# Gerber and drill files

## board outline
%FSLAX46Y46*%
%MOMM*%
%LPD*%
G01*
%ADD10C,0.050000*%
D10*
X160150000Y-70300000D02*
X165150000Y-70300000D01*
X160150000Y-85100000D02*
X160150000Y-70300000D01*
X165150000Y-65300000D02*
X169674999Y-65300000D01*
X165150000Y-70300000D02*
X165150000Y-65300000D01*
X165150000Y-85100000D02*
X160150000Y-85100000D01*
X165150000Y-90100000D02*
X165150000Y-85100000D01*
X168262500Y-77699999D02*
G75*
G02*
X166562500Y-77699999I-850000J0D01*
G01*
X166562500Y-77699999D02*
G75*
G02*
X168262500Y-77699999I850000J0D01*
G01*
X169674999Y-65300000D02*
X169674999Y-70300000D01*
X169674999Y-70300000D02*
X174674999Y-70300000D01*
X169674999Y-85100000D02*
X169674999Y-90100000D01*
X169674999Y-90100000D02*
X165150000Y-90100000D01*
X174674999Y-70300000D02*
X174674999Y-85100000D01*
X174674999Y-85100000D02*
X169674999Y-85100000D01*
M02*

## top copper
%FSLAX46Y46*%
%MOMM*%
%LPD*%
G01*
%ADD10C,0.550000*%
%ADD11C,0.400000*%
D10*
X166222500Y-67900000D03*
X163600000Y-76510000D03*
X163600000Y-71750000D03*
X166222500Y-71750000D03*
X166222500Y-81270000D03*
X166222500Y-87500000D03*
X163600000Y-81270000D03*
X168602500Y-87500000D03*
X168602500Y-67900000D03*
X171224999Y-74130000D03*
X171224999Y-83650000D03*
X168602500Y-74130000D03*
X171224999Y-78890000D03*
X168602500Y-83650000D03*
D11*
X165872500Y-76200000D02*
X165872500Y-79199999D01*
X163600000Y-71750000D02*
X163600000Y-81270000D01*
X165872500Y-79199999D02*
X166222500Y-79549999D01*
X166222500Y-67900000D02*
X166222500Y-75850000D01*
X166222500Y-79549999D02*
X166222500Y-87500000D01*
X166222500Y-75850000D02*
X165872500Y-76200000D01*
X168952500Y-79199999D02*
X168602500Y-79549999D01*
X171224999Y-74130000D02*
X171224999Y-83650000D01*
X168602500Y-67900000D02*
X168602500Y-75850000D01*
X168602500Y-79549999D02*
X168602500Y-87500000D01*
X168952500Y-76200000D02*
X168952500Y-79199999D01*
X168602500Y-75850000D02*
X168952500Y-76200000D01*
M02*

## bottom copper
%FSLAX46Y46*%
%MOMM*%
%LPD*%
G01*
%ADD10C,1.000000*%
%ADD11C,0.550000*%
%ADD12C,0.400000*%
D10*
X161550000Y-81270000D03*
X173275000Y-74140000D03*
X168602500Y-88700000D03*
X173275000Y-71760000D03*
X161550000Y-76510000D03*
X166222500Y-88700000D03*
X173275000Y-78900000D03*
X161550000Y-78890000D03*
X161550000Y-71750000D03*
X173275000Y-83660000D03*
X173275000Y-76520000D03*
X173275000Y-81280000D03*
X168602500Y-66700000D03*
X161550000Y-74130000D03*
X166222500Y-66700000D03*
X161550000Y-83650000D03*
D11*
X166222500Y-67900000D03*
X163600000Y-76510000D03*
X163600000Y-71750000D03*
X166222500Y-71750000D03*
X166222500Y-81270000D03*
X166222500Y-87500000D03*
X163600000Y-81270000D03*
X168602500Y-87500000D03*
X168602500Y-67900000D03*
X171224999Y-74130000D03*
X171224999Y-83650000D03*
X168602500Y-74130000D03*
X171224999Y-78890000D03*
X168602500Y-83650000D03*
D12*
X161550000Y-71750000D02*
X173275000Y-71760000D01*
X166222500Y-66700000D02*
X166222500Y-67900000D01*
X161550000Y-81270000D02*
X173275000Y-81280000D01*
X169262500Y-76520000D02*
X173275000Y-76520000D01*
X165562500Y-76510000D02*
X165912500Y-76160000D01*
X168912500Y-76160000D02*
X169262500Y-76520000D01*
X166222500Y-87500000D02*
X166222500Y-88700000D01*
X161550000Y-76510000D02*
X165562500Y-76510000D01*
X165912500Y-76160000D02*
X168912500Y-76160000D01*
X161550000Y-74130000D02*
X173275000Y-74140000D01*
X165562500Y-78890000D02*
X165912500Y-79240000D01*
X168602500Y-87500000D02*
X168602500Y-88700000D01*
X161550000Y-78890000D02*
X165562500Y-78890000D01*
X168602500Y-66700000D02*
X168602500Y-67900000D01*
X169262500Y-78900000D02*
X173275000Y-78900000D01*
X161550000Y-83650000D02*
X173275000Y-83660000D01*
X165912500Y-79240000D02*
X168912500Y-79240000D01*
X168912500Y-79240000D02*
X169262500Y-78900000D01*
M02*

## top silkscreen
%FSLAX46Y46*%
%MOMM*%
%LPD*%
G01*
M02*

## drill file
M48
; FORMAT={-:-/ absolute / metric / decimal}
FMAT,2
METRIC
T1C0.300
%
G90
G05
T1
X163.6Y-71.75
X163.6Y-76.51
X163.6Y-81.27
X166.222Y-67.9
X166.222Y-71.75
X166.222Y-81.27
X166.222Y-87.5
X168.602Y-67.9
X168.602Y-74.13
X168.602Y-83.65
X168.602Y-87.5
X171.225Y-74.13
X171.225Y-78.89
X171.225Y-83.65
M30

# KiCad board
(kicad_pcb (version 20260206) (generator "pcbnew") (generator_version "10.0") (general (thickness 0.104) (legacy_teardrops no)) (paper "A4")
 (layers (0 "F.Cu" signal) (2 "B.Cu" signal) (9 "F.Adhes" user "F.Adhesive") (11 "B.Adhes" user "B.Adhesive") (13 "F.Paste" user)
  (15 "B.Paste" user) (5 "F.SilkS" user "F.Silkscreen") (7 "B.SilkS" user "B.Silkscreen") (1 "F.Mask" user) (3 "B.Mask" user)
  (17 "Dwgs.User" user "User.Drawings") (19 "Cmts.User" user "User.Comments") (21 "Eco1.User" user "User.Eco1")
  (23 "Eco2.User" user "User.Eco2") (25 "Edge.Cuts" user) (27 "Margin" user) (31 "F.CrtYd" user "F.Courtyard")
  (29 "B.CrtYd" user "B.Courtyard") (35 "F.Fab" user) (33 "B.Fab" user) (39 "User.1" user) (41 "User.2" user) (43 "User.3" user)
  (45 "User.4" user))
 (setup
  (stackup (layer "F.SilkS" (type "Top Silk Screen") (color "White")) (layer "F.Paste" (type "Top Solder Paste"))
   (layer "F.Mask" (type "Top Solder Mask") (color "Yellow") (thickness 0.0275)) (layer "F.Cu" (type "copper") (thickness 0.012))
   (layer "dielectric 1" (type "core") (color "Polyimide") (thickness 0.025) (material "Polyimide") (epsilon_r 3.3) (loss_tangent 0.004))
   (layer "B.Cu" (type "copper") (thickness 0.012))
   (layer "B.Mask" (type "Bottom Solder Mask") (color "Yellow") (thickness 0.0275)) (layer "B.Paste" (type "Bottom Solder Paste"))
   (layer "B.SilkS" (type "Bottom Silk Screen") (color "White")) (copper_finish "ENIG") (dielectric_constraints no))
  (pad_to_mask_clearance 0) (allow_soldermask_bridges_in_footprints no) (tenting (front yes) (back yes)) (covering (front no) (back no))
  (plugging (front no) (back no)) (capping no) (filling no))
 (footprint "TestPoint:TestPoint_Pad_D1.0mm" (layer "B.Cu") (at 161.55 81.27 -90)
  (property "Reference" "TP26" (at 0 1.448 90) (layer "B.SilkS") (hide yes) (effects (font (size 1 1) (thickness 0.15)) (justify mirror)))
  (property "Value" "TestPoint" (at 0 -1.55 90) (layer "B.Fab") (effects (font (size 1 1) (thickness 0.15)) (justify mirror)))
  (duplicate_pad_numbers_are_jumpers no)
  (pad "1" smd circle (at 0 0 270) (size 1 1) (layers "B.Cu" "B.Mask") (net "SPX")))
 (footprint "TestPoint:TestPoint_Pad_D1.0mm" (layer "B.Cu") (at 173.275 74.14 90)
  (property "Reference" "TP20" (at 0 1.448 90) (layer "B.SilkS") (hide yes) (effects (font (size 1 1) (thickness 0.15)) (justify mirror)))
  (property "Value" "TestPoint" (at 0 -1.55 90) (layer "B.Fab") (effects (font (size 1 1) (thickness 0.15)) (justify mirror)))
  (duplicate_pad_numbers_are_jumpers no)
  (pad "1" smd circle (at 0 0 90) (size 1 1) (layers "B.Cu" "B.Mask") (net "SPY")))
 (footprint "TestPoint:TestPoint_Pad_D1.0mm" (layer "B.Cu") (at 168.6025 88.7)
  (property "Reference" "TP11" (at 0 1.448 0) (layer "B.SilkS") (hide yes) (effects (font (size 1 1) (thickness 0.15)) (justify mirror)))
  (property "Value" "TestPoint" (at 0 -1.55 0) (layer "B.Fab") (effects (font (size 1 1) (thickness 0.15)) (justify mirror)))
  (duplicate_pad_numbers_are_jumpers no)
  (pad "1" smd circle (at 0 0) (size 1 1) (layers "B.Cu" "B.Mask") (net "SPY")))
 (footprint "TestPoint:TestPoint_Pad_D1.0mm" (layer "B.Cu") (at 173.275 71.76 90)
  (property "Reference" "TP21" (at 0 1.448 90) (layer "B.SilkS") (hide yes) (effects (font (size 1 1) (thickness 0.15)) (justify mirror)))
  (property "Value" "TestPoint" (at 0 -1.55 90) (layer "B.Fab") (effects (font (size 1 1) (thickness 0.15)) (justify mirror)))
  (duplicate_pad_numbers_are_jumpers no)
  (pad "1" smd circle (at 0 0 90) (size 1 1) (layers "B.Cu" "B.Mask") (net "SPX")))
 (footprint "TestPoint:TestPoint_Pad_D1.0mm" (layer "B.Cu") (at 161.55 76.51 -90)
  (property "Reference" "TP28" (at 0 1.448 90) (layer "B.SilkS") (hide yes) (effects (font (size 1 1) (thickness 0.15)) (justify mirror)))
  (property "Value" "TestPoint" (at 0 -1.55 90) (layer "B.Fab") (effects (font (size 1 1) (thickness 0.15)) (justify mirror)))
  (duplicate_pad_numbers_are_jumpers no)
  (pad "1" smd circle (at 0 0 270) (size 1 1) (layers "B.Cu" "B.Mask") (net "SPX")))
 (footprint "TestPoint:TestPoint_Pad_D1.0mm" (layer "B.Cu") (at 166.2225 88.7)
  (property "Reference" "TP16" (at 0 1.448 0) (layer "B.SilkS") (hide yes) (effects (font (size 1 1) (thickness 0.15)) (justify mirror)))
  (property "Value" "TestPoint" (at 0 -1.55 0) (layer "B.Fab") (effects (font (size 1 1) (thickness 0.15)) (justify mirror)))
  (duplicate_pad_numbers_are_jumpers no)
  (pad "1" smd circle (at 0 0) (size 1 1) (layers "B.Cu" "B.Mask") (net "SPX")))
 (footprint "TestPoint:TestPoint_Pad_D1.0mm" (layer "B.Cu") (at 173.275 78.9 90)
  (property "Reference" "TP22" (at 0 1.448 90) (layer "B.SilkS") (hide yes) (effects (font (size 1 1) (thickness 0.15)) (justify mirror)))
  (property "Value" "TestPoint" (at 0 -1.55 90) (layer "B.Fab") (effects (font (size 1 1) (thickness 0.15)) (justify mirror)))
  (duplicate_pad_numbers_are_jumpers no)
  (pad "1" smd circle (at 0 0 90) (size 1 1) (layers "B.Cu" "B.Mask") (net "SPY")))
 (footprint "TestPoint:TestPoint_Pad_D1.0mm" (layer "B.Cu") (at 161.55 78.89 -90)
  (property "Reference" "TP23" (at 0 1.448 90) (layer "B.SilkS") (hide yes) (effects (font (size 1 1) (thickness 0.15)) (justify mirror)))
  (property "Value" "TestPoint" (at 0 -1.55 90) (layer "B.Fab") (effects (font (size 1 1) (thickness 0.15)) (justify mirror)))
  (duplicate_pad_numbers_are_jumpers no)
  (pad "1" smd circle (at 0 0 270) (size 1 1) (layers "B.Cu" "B.Mask") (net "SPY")))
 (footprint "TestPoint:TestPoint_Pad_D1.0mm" (layer "B.Cu") (at 161.55 71.75 -90)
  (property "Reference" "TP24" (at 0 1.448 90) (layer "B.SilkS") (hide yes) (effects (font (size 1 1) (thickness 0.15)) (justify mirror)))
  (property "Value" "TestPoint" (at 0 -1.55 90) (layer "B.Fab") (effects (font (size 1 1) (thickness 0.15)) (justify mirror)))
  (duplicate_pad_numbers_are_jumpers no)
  (pad "1" smd circle (at 0 0 270) (size 1 1) (layers "B.Cu" "B.Mask") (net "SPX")))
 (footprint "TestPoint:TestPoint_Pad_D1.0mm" (layer "B.Cu") (at 173.275 83.66 90)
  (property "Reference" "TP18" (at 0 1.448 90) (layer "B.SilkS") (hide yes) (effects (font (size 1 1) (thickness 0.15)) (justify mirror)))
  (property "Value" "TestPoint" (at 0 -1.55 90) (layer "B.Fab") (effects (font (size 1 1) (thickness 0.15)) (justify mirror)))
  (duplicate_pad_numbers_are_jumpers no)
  (pad "1" smd circle (at 0 0 90) (size 1 1) (layers "B.Cu" "B.Mask") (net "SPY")))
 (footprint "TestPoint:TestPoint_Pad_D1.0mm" (layer "B.Cu") (at 173.275 76.52 90)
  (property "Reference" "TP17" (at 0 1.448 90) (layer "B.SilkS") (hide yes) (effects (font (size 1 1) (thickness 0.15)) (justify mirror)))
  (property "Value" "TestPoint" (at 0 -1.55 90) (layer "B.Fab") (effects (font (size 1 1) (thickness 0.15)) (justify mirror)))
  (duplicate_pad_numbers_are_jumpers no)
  (pad "1" smd circle (at 0 0 90) (size 1 1) (layers "B.Cu" "B.Mask") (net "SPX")))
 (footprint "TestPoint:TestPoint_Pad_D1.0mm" (layer "B.Cu") (at 173.275 81.28 90)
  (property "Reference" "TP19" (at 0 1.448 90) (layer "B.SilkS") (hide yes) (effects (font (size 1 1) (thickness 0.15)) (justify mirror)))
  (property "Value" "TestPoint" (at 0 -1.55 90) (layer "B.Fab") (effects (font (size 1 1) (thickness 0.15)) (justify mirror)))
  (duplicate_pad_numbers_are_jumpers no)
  (pad "1" smd circle (at 0 0 90) (size 1 1) (layers "B.Cu" "B.Mask") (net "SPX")))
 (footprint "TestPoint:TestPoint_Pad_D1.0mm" (layer "B.Cu") (at 168.6025 66.7 180)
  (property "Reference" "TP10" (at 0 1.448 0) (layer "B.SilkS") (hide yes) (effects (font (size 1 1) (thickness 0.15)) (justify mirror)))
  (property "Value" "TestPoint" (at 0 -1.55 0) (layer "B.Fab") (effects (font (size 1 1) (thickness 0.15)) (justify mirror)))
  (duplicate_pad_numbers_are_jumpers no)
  (pad "1" smd circle (at 0 0 180) (size 1 1) (layers "B.Cu" "B.Mask") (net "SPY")))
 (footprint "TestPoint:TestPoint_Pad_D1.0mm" (layer "B.Cu") (at 161.55 74.13 -90)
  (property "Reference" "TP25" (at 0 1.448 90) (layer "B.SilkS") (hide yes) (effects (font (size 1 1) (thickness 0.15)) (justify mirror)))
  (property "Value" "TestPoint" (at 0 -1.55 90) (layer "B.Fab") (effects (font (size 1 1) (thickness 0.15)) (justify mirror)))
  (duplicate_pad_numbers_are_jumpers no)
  (pad "1" smd circle (at 0 0 270) (size 1 1) (layers "B.Cu" "B.Mask") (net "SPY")))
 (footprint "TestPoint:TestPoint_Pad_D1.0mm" (layer "B.Cu") (at 166.2225 66.7 180)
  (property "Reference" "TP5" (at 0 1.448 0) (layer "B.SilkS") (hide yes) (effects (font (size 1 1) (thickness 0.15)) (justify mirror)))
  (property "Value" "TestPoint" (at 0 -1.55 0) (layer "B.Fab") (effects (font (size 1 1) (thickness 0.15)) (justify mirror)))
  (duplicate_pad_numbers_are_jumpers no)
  (pad "1" smd circle (at 0 0 180) (size 1 1) (layers "B.Cu" "B.Mask") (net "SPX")))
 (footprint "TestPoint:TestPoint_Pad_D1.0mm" (layer "B.Cu") (at 161.55 83.65 -90)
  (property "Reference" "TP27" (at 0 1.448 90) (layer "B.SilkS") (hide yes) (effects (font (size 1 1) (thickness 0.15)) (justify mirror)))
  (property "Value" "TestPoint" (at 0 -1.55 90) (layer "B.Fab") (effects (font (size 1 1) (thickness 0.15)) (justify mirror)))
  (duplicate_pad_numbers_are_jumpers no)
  (pad "1" smd circle (at 0 0 270) (size 1 1) (layers "B.Cu" "B.Mask") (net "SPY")))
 (gr_line (start 160.15 70.3) (end 165.15 70.3) (stroke (width 0.05) (type default)) (layer "Edge.Cuts"))
 (gr_line (start 160.15 85.1) (end 160.15 70.3) (stroke (width 0.05) (type default)) (layer "Edge.Cuts"))
 (gr_line (start 165.15 65.3) (end 169.674999 65.3) (stroke (width 0.05) (type default)) (layer "Edge.Cuts"))
 (gr_line (start 165.15 70.3) (end 165.15 65.3) (stroke (width 0.05) (type default)) (layer "Edge.Cuts"))
 (gr_line (start 165.15 85.1) (end 160.15 85.1) (stroke (width 0.05) (type default)) (layer "Edge.Cuts"))
 (gr_line (start 165.15 90.1) (end 165.15 85.1) (stroke (width 0.05) (type default)) (layer "Edge.Cuts"))
 (gr_circle (center 167.4125 77.699999) (end 168.2625 77.699999) (stroke (width 0.05) (type default)) (fill no) (layer "Edge.Cuts"))
 (gr_line (start 169.674999 65.3) (end 169.674999 70.3) (stroke (width 0.05) (type default)) (layer "Edge.Cuts"))
 (gr_line (start 169.674999 70.3) (end 174.674999 70.3) (stroke (width 0.05) (type default)) (layer "Edge.Cuts"))
 (gr_line (start 169.674999 85.1) (end 169.674999 90.1) (stroke (width 0.05) (type default)) (layer "Edge.Cuts"))
 (gr_line (start 169.674999 90.1) (end 165.15 90.1) (stroke (width 0.05) (type default)) (layer "Edge.Cuts"))
 (gr_line (start 174.674999 70.3) (end 174.674999 85.1) (stroke (width 0.05) (type default)) (layer "Edge.Cuts"))
 (gr_line (start 174.674999 85.1) (end 169.674999 85.1) (stroke (width 0.05) (type default)) (layer "Edge.Cuts"))
 (segment (start 165.8725 76.2) (end 165.8725 79.199999) (width 0.4) (layer "F.Cu") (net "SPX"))
 (segment (start 163.6 71.75) (end 163.6 81.27) (width 0.4) (layer "F.Cu") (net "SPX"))
 (segment (start 165.8725 79.199999) (end 166.2225 79.549999) (width 0.4) (layer "F.Cu") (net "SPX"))
 (segment (start 166.2225 67.9) (end 166.2225 75.85) (width 0.4) (layer "F.Cu") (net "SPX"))
 (segment (start 166.2225 79.549999) (end 166.2225 87.5) (width 0.4) (layer "F.Cu") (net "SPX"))
 (segment (start 166.2225 75.85) (end 165.8725 76.2) (width 0.4) (layer "F.Cu") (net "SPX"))
 (via (at 166.2225 67.9) (size 0.55) (drill 0.3) (layers "F.Cu" "B.Cu") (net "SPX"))
 (via (at 163.6 76.51) (size 0.55) (drill 0.3) (layers "F.Cu" "B.Cu") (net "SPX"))
 (via (at 163.6 71.75) (size 0.55) (drill 0.3) (layers "F.Cu" "B.Cu") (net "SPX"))
 (via (at 166.2225 71.75) (size 0.55) (drill 0.3) (layers "F.Cu" "B.Cu") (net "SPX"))
 (via (at 166.2225 81.27) (size 0.55) (drill 0.3) (layers "F.Cu" "B.Cu") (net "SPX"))
 (via (at 166.2225 87.5) (size 0.55) (drill 0.3) (layers "F.Cu" "B.Cu") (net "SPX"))
 (via (at 163.6 81.27) (size 0.55) (drill 0.3) (layers "F.Cu" "B.Cu") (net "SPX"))
 (segment (start 161.55 71.75) (end 173.275 71.76) (width 0.4) (layer "B.Cu") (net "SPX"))
 (segment (start 166.2225 66.7) (end 166.2225 67.9) (width 0.4) (layer "B.Cu") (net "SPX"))
 (segment (start 161.55 81.27) (end 173.275 81.28) (width 0.4) (layer "B.Cu") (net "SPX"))
 (segment (start 169.2625 76.52) (end 173.275 76.52) (width 0.4) (layer "B.Cu") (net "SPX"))
 (segment (start 165.5625 76.51) (end 165.9125 76.16) (width 0.4) (layer "B.Cu") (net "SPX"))
 (segment (start 168.9125 76.16) (end 169.2625 76.52) (width 0.4) (layer "B.Cu") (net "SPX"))
 (segment (start 166.2225 87.5) (end 166.2225 88.7) (width 0.4) (layer "B.Cu") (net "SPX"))
 (segment (start 161.55 76.51) (end 165.5625 76.51) (width 0.4) (layer "B.Cu") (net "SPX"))
 (segment (start 165.9125 76.16) (end 168.9125 76.16) (width 0.4) (layer "B.Cu") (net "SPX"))
 (segment (start 168.9525 79.199999) (end 168.6025 79.549999) (width 0.4) (layer "F.Cu") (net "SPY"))
 (segment (start 171.224999 74.13) (end 171.224999 83.65) (width 0.4) (layer "F.Cu") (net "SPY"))
 (segment (start 168.6025 67.9) (end 168.6025 75.85) (width 0.4) (layer "F.Cu") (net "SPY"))
 (segment (start 168.6025 79.549999) (end 168.6025 87.5) (width 0.4) (layer "F.Cu") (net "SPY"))
 (segment (start 168.9525 76.2) (end 168.9525 79.199999) (width 0.4) (layer "F.Cu") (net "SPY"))
 (segment (start 168.6025 75.85) (end 168.9525 76.2) (width 0.4) (layer "F.Cu") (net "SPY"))
 (via (at 168.6025 87.5) (size 0.55) (drill 0.3) (layers "F.Cu" "B.Cu") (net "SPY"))
 (via (at 168.6025 67.9) (size 0.55) (drill 0.3) (layers "F.Cu" "B.Cu") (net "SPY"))
 (via (at 171.224999 74.13) (size 0.55) (drill 0.3) (layers "F.Cu" "B.Cu") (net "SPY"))
 (via (at 171.224999 83.65) (size 0.55) (drill 0.3) (layers "F.Cu" "B.Cu") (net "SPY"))
 (via (at 168.6025 74.13) (size 0.55) (drill 0.3) (layers "F.Cu" "B.Cu") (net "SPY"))
 (via (at 171.224999 78.89) (size 0.55) (drill 0.3) (layers "F.Cu" "B.Cu") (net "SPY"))
 (via (at 168.6025 83.65) (size 0.55) (drill 0.3) (layers "F.Cu" "B.Cu") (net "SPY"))
 (segment (start 161.55 74.13) (end 173.275 74.14) (width 0.4) (layer "B.Cu") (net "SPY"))
 (segment (start 165.5625 78.89) (end 165.9125 79.24) (width 0.4) (layer "B.Cu") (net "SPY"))
 (segment (start 168.6025 87.5) (end 168.6025 88.7) (width 0.4) (layer "B.Cu") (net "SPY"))
 (segment (start 161.55 78.89) (end 165.5625 78.89) (width 0.4) (layer "B.Cu") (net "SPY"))
 (segment (start 168.6025 66.7) (end 168.6025 67.9) (width 0.4) (layer "B.Cu") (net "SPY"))
 (segment (start 169.2625 78.9) (end 173.275 78.9) (width 0.4) (layer "B.Cu") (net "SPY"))
 (segment (start 161.55 83.65) (end 173.275 83.66) (width 0.4) (layer "B.Cu") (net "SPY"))
 (segment (start 165.9125 79.24) (end 168.9125 79.24) (width 0.4) (layer "B.Cu") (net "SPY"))
 (segment (start 168.9125 79.24) (end 169.2625 78.9) (width 0.4) (layer "B.Cu") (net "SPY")))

